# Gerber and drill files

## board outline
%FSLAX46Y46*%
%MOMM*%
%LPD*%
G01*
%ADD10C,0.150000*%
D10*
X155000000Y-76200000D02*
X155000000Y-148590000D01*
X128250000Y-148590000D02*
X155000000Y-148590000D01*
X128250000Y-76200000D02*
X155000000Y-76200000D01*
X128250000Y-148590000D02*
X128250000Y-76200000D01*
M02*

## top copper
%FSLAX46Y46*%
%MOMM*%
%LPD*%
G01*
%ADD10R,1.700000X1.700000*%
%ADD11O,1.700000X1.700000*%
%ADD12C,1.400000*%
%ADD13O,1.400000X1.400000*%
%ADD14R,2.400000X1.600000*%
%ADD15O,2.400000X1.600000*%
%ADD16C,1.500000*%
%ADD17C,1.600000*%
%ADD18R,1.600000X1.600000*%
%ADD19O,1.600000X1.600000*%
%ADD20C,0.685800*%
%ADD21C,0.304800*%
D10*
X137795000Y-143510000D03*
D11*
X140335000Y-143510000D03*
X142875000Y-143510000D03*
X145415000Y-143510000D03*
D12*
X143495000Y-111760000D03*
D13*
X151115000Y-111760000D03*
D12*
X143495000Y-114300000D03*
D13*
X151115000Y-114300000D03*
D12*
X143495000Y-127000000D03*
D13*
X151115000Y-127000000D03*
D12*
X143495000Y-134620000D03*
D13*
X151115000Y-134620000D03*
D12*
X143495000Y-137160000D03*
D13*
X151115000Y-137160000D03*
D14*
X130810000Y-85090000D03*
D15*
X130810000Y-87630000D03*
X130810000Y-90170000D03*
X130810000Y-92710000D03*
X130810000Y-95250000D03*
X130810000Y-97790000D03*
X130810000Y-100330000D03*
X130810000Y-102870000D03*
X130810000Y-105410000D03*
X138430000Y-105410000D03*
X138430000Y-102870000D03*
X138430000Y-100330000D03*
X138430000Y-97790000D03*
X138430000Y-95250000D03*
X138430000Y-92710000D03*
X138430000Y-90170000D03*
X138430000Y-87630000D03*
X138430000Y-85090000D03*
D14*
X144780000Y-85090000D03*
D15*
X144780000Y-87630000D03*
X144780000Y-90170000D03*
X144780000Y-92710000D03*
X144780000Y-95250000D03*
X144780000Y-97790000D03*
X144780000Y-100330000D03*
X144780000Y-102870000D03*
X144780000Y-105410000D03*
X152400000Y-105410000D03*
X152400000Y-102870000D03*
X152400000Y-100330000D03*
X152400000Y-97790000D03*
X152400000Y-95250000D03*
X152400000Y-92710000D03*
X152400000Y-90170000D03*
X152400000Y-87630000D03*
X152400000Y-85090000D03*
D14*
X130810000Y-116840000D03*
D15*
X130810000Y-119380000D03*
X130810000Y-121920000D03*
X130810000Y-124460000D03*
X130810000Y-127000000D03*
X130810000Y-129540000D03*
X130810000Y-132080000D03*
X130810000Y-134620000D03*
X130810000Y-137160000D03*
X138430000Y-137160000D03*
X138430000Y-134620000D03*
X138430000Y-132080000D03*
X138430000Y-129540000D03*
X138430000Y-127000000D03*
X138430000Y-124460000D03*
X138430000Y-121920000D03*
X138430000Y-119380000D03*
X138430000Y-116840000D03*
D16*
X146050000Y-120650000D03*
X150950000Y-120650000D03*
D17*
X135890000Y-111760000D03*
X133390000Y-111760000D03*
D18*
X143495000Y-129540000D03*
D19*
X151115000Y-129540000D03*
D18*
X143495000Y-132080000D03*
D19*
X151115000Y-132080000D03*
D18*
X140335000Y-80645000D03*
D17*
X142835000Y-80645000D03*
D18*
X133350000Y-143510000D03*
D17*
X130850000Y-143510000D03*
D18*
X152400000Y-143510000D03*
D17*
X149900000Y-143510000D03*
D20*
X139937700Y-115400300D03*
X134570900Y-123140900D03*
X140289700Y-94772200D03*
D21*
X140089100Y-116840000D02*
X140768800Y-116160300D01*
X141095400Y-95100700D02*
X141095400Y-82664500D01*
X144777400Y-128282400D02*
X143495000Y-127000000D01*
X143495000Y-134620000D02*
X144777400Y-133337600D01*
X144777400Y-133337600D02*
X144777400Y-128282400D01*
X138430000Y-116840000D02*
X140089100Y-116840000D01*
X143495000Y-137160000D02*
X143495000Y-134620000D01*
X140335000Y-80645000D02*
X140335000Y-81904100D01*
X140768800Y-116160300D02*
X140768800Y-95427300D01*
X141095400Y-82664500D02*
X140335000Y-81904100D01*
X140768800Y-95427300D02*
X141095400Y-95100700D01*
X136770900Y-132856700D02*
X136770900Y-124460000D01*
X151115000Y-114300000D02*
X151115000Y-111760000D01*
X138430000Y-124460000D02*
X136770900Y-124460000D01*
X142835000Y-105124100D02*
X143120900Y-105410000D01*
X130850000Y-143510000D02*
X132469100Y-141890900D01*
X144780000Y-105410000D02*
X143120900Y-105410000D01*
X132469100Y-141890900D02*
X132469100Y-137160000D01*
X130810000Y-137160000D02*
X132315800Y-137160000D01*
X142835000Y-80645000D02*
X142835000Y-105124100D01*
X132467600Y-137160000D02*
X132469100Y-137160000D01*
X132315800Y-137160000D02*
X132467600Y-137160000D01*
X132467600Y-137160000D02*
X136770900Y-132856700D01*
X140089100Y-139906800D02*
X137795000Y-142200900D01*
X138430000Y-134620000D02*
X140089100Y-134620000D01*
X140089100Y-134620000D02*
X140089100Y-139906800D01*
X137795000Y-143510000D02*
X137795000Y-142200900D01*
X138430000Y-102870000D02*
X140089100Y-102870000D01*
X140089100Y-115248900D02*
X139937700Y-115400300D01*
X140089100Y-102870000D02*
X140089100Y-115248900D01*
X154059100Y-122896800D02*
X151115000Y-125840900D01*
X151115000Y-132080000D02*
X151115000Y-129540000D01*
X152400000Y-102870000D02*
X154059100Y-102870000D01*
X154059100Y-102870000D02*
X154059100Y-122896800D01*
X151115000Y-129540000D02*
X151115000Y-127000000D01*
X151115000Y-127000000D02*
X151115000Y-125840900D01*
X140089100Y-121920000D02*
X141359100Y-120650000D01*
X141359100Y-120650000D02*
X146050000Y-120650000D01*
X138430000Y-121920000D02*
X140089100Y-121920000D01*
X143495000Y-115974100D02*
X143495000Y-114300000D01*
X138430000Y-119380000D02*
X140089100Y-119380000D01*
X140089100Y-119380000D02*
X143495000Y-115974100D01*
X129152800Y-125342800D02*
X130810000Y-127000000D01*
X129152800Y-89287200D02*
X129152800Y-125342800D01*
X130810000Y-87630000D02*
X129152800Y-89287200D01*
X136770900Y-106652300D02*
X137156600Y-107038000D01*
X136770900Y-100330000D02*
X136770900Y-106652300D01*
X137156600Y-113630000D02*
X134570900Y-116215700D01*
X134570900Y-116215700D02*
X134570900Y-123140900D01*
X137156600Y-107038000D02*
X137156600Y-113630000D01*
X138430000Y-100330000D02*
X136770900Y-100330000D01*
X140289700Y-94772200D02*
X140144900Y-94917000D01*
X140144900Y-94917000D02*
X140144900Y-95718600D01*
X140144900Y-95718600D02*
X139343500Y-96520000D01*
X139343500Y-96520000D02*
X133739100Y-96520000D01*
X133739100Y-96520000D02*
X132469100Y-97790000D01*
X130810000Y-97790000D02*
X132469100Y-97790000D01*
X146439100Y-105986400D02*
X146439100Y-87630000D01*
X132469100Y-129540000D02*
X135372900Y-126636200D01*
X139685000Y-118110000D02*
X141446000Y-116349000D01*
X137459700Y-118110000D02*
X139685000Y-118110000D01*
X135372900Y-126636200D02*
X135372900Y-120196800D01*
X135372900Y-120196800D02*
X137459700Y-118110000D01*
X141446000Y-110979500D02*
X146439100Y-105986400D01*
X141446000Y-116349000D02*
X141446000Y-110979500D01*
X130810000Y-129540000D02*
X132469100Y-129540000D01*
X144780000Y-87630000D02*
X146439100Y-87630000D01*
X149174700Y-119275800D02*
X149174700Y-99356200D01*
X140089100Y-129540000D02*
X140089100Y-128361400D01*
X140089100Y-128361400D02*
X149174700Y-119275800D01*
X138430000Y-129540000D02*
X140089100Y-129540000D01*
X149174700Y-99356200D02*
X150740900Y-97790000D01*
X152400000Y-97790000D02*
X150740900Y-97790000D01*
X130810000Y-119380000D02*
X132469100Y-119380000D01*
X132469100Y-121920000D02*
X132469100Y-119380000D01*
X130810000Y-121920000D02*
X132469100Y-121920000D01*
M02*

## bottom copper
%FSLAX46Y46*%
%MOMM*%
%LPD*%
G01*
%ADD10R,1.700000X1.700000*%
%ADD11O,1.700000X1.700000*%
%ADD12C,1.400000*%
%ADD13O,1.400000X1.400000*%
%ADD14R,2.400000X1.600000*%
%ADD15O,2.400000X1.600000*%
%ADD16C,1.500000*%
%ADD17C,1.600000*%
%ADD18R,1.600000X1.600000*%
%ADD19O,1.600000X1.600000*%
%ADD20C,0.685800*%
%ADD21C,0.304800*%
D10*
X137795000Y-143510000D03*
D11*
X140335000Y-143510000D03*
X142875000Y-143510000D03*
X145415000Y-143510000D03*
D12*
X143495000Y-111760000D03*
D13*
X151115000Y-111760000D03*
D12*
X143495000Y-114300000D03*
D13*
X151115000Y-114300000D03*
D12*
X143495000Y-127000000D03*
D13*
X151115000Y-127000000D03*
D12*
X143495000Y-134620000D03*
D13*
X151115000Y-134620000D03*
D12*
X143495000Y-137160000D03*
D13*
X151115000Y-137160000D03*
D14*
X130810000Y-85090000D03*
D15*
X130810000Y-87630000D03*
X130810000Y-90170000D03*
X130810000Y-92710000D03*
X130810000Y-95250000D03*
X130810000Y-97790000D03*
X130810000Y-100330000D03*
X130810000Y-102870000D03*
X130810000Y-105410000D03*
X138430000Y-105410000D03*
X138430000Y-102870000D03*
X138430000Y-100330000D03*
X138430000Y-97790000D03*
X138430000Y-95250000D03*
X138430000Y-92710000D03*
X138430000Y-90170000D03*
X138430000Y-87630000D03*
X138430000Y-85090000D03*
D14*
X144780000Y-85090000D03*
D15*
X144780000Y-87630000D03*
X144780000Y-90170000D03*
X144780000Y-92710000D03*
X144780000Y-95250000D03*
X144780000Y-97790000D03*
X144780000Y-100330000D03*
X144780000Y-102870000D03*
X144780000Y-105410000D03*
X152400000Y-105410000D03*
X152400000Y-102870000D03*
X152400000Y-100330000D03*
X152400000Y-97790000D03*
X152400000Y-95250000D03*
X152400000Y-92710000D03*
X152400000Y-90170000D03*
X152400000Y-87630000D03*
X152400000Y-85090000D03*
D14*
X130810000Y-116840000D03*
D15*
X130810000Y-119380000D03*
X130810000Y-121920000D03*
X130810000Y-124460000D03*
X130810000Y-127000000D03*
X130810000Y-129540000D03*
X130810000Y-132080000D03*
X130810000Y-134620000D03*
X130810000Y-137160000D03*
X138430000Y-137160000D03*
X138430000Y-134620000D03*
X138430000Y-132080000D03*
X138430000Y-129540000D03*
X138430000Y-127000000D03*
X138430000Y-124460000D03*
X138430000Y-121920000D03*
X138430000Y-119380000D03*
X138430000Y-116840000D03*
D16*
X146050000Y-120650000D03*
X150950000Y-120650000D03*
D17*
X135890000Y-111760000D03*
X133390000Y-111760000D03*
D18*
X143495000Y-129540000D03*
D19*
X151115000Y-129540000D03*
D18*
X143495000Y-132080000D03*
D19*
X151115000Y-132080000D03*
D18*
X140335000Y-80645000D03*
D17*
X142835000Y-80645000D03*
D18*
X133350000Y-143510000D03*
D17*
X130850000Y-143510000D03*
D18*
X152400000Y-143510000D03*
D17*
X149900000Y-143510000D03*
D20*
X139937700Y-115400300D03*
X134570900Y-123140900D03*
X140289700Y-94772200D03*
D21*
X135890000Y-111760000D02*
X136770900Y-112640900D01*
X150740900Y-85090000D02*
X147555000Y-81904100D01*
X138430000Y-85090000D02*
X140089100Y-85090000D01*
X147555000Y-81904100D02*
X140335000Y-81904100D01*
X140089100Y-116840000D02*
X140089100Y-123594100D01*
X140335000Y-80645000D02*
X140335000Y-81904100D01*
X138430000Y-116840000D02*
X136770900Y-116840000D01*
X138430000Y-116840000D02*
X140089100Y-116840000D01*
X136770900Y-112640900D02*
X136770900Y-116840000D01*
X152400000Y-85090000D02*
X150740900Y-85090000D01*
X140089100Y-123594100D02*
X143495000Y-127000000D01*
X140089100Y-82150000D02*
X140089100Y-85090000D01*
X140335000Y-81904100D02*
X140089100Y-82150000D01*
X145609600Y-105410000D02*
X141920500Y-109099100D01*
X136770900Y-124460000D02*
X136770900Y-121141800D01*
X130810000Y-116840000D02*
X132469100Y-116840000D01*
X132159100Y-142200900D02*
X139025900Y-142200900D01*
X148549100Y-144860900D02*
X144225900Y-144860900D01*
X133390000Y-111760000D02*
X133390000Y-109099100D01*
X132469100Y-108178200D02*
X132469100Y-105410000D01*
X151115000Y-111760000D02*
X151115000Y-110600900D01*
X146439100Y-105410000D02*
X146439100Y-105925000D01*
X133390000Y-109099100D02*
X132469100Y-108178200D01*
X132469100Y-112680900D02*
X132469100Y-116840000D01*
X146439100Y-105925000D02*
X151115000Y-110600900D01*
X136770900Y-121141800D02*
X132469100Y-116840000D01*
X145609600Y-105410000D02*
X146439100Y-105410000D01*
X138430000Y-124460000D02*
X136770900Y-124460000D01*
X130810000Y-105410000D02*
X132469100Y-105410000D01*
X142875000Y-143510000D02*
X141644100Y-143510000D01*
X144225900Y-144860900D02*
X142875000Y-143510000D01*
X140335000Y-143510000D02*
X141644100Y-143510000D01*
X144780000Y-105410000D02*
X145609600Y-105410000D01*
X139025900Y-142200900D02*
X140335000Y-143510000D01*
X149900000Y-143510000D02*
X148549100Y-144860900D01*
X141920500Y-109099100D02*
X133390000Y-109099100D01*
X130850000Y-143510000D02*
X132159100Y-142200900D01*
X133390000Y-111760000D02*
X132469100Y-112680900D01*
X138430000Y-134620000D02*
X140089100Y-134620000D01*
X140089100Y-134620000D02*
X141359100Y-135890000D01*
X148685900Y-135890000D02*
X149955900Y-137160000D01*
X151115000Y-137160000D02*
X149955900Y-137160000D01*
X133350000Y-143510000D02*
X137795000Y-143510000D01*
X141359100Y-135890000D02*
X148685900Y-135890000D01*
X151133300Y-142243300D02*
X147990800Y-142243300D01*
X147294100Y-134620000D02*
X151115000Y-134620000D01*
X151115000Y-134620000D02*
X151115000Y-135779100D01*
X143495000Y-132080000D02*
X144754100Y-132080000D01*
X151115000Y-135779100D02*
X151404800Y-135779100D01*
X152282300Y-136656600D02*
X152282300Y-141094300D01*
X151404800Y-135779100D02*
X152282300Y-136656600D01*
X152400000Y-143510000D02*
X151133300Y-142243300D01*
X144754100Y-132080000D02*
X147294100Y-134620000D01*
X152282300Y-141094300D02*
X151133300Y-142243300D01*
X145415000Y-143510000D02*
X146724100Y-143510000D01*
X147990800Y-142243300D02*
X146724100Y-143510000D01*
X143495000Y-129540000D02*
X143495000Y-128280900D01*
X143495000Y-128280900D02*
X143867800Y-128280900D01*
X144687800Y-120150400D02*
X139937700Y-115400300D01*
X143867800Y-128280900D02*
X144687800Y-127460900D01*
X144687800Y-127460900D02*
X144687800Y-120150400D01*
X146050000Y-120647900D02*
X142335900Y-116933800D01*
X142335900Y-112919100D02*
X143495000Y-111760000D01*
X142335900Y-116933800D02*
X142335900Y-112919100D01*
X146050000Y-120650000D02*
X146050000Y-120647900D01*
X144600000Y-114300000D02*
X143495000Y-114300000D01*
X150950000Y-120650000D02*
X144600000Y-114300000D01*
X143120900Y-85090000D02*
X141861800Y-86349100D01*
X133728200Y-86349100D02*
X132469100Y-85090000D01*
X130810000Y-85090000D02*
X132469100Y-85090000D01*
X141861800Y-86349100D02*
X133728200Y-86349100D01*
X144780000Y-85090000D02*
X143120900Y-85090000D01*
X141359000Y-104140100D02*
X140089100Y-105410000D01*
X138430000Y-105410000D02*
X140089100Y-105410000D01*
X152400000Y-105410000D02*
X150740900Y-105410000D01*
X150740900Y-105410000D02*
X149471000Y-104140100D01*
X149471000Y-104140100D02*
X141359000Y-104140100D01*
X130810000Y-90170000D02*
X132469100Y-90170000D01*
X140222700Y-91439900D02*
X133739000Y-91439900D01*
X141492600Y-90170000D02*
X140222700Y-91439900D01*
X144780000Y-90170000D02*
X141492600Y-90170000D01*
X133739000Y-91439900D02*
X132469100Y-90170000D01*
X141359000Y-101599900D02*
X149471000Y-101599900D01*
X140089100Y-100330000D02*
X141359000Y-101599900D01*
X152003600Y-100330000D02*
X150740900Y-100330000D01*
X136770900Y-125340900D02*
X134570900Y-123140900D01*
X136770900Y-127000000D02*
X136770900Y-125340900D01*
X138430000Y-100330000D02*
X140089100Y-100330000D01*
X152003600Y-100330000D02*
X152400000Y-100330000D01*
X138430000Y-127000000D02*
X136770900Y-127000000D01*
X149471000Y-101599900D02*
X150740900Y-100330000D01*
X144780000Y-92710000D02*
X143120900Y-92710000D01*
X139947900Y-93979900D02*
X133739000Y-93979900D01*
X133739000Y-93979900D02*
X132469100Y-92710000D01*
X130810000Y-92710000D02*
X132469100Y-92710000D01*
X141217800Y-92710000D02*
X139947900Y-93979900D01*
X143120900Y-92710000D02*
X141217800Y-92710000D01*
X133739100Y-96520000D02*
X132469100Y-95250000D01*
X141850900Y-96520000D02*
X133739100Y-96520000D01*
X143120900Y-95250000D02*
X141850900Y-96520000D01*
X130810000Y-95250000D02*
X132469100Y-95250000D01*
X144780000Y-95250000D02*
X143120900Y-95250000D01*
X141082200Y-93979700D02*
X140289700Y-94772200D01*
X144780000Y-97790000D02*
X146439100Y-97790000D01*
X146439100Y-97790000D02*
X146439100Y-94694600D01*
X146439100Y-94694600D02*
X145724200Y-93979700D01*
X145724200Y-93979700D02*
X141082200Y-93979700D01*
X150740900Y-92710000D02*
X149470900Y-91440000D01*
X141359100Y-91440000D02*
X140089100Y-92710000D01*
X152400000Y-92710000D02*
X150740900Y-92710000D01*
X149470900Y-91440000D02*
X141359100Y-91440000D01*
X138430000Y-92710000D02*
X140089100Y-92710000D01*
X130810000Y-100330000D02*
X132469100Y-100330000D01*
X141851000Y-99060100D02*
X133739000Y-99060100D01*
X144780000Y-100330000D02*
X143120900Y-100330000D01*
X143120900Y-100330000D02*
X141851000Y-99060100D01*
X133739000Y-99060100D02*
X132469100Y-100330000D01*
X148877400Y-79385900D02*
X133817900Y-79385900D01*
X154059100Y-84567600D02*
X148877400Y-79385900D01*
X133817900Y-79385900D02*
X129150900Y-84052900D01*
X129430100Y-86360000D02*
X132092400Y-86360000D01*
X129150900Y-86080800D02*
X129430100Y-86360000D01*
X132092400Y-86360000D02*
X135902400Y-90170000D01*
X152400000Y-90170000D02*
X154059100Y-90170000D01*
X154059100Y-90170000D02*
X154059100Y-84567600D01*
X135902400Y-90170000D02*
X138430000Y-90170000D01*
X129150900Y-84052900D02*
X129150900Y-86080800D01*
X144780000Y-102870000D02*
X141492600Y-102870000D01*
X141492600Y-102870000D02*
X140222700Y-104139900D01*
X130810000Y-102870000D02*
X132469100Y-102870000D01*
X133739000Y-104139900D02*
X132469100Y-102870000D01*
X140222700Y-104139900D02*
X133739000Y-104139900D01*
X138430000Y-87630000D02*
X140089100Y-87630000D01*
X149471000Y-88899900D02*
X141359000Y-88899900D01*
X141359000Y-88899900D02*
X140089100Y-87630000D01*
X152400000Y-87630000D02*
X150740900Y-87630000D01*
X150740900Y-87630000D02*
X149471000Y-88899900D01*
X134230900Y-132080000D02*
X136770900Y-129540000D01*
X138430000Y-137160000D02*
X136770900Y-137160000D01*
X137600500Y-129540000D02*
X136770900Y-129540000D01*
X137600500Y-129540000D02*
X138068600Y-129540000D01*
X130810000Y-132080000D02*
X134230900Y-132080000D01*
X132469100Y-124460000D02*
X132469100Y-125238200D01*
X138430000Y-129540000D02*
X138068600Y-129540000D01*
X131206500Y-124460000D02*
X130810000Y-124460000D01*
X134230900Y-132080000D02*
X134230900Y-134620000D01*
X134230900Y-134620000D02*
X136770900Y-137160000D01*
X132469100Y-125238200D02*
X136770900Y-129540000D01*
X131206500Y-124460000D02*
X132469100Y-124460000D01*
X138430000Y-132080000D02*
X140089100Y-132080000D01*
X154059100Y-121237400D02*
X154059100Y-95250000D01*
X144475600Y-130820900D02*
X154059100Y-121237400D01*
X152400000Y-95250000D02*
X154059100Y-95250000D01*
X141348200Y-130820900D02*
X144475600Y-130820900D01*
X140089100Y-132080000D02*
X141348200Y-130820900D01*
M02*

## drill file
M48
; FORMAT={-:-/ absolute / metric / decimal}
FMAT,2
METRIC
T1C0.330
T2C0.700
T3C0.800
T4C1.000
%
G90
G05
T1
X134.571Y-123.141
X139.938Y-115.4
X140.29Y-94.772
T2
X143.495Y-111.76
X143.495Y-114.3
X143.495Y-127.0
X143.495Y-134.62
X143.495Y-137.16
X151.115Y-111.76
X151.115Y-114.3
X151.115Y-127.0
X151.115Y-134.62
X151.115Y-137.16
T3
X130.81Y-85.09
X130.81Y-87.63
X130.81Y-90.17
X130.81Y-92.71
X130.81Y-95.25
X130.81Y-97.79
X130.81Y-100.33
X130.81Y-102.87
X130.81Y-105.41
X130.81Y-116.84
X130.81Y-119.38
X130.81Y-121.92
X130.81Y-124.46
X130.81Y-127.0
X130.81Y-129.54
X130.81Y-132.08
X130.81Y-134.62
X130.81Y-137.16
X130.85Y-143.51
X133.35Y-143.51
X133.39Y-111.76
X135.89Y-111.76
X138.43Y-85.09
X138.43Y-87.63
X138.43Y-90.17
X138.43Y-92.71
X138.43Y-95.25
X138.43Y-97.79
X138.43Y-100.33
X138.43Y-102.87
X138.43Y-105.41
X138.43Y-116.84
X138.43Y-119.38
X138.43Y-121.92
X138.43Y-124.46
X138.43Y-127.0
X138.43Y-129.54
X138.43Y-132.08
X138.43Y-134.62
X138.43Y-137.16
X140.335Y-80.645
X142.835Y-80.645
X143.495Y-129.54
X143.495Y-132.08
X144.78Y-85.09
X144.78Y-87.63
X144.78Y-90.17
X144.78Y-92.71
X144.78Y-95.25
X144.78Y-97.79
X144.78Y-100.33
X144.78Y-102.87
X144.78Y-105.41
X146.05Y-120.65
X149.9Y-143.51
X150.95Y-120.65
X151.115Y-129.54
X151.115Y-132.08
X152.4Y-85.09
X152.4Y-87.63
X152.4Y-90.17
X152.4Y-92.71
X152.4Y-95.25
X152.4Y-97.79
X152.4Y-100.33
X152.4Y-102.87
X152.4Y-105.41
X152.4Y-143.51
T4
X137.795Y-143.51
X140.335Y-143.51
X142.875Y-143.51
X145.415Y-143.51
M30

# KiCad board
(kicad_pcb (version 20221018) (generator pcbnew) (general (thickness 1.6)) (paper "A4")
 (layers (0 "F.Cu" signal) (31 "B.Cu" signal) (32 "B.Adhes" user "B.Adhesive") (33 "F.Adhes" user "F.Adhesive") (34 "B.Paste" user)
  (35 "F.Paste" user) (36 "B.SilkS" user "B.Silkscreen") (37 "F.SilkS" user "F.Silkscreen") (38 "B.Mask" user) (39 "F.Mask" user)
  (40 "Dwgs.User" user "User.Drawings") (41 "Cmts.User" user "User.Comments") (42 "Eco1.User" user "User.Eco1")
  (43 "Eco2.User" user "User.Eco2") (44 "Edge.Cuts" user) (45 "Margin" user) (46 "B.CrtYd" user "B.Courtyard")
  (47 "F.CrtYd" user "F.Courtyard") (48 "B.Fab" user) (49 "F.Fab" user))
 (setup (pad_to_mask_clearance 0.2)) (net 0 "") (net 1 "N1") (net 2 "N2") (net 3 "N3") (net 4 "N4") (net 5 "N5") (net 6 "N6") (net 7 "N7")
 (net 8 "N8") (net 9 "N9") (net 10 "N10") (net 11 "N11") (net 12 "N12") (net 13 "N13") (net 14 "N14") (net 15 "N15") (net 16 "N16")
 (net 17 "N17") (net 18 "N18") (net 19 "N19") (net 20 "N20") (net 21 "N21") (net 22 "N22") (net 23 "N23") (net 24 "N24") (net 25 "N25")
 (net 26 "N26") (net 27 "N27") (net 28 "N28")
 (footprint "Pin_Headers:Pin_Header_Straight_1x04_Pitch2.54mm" (layer "F.Cu") (at 137.795 143.51 90)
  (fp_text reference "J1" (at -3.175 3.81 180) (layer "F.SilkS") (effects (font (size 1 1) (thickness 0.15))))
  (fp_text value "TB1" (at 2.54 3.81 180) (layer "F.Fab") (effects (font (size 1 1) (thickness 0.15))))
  (pad "1" thru_hole rect (at 0 0 90) (size 1.7 1.7) (drill 1) (layers "*.Cu" "*.Mask") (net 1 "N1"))
  (pad "2" thru_hole oval (at 0 2.54 90) (size 1.7 1.7) (drill 1) (layers "*.Cu" "*.Mask") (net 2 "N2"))
  (pad "3" thru_hole oval (at 0 5.08 90) (size 1.7 1.7) (drill 1) (layers "*.Cu" "*.Mask") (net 2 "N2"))
  (pad "4" thru_hole oval (at 0 7.62 90) (size 1.7 1.7) (drill 1) (layers "*.Cu" "*.Mask") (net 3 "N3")))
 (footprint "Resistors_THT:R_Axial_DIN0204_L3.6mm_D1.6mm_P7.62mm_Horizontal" (layer "F.Cu") (at 143.495 111.76)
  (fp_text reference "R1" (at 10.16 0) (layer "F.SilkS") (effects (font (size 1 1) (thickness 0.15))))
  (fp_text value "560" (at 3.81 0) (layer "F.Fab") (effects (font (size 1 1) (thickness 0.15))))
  (pad "1" thru_hole circle (at 0 0) (size 1.4 1.4) (drill 0.7) (layers "*.Cu" "*.Mask") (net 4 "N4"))
  (pad "2" thru_hole oval (at 7.62 0) (size 1.4 1.4) (drill 0.7) (layers "*.Cu" "*.Mask") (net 2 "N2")))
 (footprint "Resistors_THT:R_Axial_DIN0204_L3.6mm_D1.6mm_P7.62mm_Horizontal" (layer "F.Cu") (at 143.495 114.3)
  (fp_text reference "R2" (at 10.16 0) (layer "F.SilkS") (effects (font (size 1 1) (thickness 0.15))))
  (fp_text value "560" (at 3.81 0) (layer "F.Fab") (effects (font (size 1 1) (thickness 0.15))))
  (pad "1" thru_hole circle (at 0 0) (size 1.4 1.4) (drill 0.7) (layers "*.Cu" "*.Mask") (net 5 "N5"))
  (pad "2" thru_hole oval (at 7.62 0) (size 1.4 1.4) (drill 0.7) (layers "*.Cu" "*.Mask") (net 2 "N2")))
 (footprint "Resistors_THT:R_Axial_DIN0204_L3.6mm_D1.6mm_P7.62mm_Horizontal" (layer "F.Cu") (at 143.495 127)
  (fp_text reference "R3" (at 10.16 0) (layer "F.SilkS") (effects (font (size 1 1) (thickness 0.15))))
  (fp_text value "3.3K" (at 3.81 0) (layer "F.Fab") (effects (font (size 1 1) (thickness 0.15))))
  (pad "1" thru_hole circle (at 0 0) (size 1.4 1.4) (drill 0.7) (layers "*.Cu" "*.Mask") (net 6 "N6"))
  (pad "2" thru_hole oval (at 7.62 0) (size 1.4 1.4) (drill 0.7) (layers "*.Cu" "*.Mask") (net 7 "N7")))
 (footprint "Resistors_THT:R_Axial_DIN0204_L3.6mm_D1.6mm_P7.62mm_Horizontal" (layer "F.Cu") (at 143.495 134.62)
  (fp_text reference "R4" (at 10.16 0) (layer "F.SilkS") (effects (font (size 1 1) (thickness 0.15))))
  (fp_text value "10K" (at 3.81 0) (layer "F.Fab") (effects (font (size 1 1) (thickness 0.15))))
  (pad "1" thru_hole circle (at 0 0) (size 1.4 1.4) (drill 0.7) (layers "*.Cu" "*.Mask") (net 6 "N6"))
  (pad "2" thru_hole oval (at 7.62 0) (size 1.4 1.4) (drill 0.7) (layers "*.Cu" "*.Mask") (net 3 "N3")))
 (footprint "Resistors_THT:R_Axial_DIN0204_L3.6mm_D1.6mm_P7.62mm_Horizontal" (layer "F.Cu") (at 143.495 137.16)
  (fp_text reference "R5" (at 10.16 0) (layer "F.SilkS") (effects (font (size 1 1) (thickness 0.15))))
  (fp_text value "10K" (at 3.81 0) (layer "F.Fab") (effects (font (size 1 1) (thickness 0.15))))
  (pad "1" thru_hole circle (at 0 0) (size 1.4 1.4) (drill 0.7) (layers "*.Cu" "*.Mask") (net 6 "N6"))
  (pad "2" thru_hole oval (at 7.62 0) (size 1.4 1.4) (drill 0.7) (layers "*.Cu" "*.Mask") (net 1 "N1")))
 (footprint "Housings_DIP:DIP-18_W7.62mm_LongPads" (layer "F.Cu") (at 130.81 85.09)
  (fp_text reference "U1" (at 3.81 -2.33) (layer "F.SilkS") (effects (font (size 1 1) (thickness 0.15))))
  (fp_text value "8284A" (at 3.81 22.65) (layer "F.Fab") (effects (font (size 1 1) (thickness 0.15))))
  (pad "1" thru_hole rect (at 0 0) (size 2.4 1.6) (drill 0.8) (layers "*.Cu" "*.Mask") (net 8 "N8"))
  (pad "2" thru_hole oval (at 0 2.54) (size 2.4 1.6) (drill 0.8) (layers "*.Cu" "*.Mask") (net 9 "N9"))
  (pad "3" thru_hole oval (at 0 5.08) (size 2.4 1.6) (drill 0.8) (layers "*.Cu" "*.Mask") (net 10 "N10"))
  (pad "4" thru_hole oval (at 0 7.62) (size 2.4 1.6) (drill 0.8) (layers "*.Cu" "*.Mask") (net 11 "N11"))
  (pad "5" thru_hole oval (at 0 10.16) (size 2.4 1.6) (drill 0.8) (layers "*.Cu" "*.Mask") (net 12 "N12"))
  (pad "6" thru_hole oval (at 0 12.7) (size 2.4 1.6) (drill 0.8) (layers "*.Cu" "*.Mask") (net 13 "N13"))
  (pad "7" thru_hole oval (at 0 15.24) (size 2.4 1.6) (drill 0.8) (layers "*.Cu" "*.Mask") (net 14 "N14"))
  (pad "8" thru_hole oval (at 0 17.78) (size 2.4 1.6) (drill 0.8) (layers "*.Cu" "*.Mask") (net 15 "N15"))
  (pad "9" thru_hole oval (at 0 20.32) (size 2.4 1.6) (drill 0.8) (layers "*.Cu" "*.Mask") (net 2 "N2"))
  (pad "10" thru_hole oval (at 7.62 20.32) (size 2.4 1.6) (drill 0.8) (layers "*.Cu" "*.Mask") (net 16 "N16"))
  (pad "11" thru_hole oval (at 7.62 17.78) (size 2.4 1.6) (drill 0.8) (layers "*.Cu" "*.Mask") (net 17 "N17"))
  (pad "12" thru_hole oval (at 7.62 15.24) (size 2.4 1.6) (drill 0.8) (layers "*.Cu" "*.Mask") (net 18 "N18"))
  (pad "13" thru_hole oval (at 7.62 12.7) (size 2.4 1.6) (drill 0.8) (layers "*.Cu" "*.Mask") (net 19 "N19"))
  (pad "14" thru_hole oval (at 7.62 10.16) (size 2.4 1.6) (drill 0.8) (layers "*.Cu" "*.Mask") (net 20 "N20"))
  (pad "15" thru_hole oval (at 7.62 7.62) (size 2.4 1.6) (drill 0.8) (layers "*.Cu" "*.Mask") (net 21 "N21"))
  (pad "16" thru_hole oval (at 7.62 5.08) (size 2.4 1.6) (drill 0.8) (layers "*.Cu" "*.Mask") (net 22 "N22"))
  (pad "17" thru_hole oval (at 7.62 2.54) (size 2.4 1.6) (drill 0.8) (layers "*.Cu" "*.Mask") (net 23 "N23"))
  (pad "18" thru_hole oval (at 7.62 0) (size 2.4 1.6) (drill 0.8) (layers "*.Cu" "*.Mask") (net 6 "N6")))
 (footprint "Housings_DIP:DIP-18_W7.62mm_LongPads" (layer "F.Cu") (at 144.78 85.09)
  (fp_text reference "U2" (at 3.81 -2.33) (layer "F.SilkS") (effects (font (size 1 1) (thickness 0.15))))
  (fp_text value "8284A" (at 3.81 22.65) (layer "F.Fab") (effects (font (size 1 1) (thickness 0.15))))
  (pad "1" thru_hole rect (at 0 0) (size 2.4 1.6) (drill 0.8) (layers "*.Cu" "*.Mask") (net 8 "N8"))
  (pad "2" thru_hole oval (at 0 2.54) (size 2.4 1.6) (drill 0.8) (layers "*.Cu" "*.Mask") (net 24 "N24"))
  (pad "3" thru_hole oval (at 0 5.08) (size 2.4 1.6) (drill 0.8) (layers "*.Cu" "*.Mask") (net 10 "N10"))
  (pad "4" thru_hole oval (at 0 7.62) (size 2.4 1.6) (drill 0.8) (layers "*.Cu" "*.Mask") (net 11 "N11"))
  (pad "5" thru_hole oval (at 0 10.16) (size 2.4 1.6) (drill 0.8) (layers "*.Cu" "*.Mask") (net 12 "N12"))
  (pad "6" thru_hole oval (at 0 12.7) (size 2.4 1.6) (drill 0.8) (layers "*.Cu" "*.Mask") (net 13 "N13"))
  (pad "7" thru_hole oval (at 0 15.24) (size 2.4 1.6) (drill 0.8) (layers "*.Cu" "*.Mask") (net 14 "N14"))
  (pad "8" thru_hole oval (at 0 17.78) (size 2.4 1.6) (drill 0.8) (layers "*.Cu" "*.Mask") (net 15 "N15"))
  (pad "9" thru_hole oval (at 0 20.32) (size 2.4 1.6) (drill 0.8) (layers "*.Cu" "*.Mask") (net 2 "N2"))
  (pad "10" thru_hole oval (at 7.62 20.32) (size 2.4 1.6) (drill 0.8) (layers "*.Cu" "*.Mask") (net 16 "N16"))
  (pad "11" thru_hole oval (at 7.62 17.78) (size 2.4 1.6) (drill 0.8) (layers "*.Cu" "*.Mask") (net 7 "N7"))
  (pad "12" thru_hole oval (at 7.62 15.24) (size 2.4 1.6) (drill 0.8) (layers "*.Cu" "*.Mask") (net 18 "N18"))
  (pad "13" thru_hole oval (at 7.62 12.7) (size 2.4 1.6) (drill 0.8) (layers "*.Cu" "*.Mask") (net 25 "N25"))
  (pad "14" thru_hole oval (at 7.62 10.16) (size 2.4 1.6) (drill 0.8) (layers "*.Cu" "*.Mask") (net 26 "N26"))
  (pad "15" thru_hole oval (at 7.62 7.62) (size 2.4 1.6) (drill 0.8) (layers "*.Cu" "*.Mask") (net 21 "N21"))
  (pad "16" thru_hole oval (at 7.62 5.08) (size 2.4 1.6) (drill 0.8) (layers "*.Cu" "*.Mask") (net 22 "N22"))
  (pad "17" thru_hole oval (at 7.62 2.54) (size 2.4 1.6) (drill 0.8) (layers "*.Cu" "*.Mask") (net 23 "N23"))
  (pad "18" thru_hole oval (at 7.62 0) (size 2.4 1.6) (drill 0.8) (layers "*.Cu" "*.Mask") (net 6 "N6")))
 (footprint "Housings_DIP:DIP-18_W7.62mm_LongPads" (layer "F.Cu") (at 130.81 116.84)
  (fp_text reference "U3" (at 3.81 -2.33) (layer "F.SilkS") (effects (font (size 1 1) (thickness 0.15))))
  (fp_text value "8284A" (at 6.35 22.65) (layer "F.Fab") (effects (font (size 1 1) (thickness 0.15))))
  (pad "1" thru_hole rect (at 0 0) (size 2.4 1.6) (drill 0.8) (layers "*.Cu" "*.Mask") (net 2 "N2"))
  (pad "2" thru_hole oval (at 0 2.54) (size 2.4 1.6) (drill 0.8) (layers "*.Cu" "*.Mask") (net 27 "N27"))
  (pad "3" thru_hole oval (at 0 5.08) (size 2.4 1.6) (drill 0.8) (layers "*.Cu" "*.Mask") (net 27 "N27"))
  (pad "4" thru_hole oval (at 0 7.62) (size 2.4 1.6) (drill 0.8) (layers "*.Cu" "*.Mask") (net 25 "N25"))
  (pad "5" thru_hole oval (at 0 10.16) (size 2.4 1.6) (drill 0.8) (layers "*.Cu" "*.Mask") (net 9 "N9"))
  (pad "6" thru_hole oval (at 0 12.7) (size 2.4 1.6) (drill 0.8) (layers "*.Cu" "*.Mask") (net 24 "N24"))
  (pad "7" thru_hole oval (at 0 15.24) (size 2.4 1.6) (drill 0.8) (layers "*.Cu" "*.Mask") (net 25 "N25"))
  (pad "8" thru_hole oval (at 0 17.78) (size 2.4 1.6) (drill 0.8) (layers "*.Cu" "*.Mask") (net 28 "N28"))
  (pad "9" thru_hole oval (at 0 20.32) (size 2.4 1.6) (drill 0.8) (layers "*.Cu" "*.Mask") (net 2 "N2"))
  (pad "10" thru_hole oval (at 7.62 20.32) (size 2.4 1.6) (drill 0.8) (layers "*.Cu" "*.Mask") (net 25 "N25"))
  (pad "11" thru_hole oval (at 7.62 17.78) (size 2.4 1.6) (drill 0.8) (layers "*.Cu" "*.Mask") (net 1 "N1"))
  (pad "12" thru_hole oval (at 7.62 15.24) (size 2.4 1.6) (drill 0.8) (layers "*.Cu" "*.Mask") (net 26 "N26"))
  (pad "13" thru_hole oval (at 7.62 12.7) (size 2.4 1.6) (drill 0.8) (layers "*.Cu" "*.Mask") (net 25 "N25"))
  (pad "14" thru_hole oval (at 7.62 10.16) (size 2.4 1.6) (drill 0.8) (layers "*.Cu" "*.Mask") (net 18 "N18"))
  (pad "15" thru_hole oval (at 7.62 7.62) (size 2.4 1.6) (drill 0.8) (layers "*.Cu" "*.Mask") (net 2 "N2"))
  (pad "16" thru_hole oval (at 7.62 5.08) (size 2.4 1.6) (drill 0.8) (layers "*.Cu" "*.Mask") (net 4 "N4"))
  (pad "17" thru_hole oval (at 7.62 2.54) (size 2.4 1.6) (drill 0.8) (layers "*.Cu" "*.Mask") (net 5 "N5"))
  (pad "18" thru_hole oval (at 7.62 0) (size 2.4 1.6) (drill 0.8) (layers "*.Cu" "*.Mask") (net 6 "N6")))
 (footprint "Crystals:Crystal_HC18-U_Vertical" (layer "F.Cu") (at 146.05 120.65)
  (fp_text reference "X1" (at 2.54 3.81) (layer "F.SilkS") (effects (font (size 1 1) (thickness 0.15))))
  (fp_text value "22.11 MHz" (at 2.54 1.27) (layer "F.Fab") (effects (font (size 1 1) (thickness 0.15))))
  (pad "1" thru_hole circle (at 0 0) (size 1.5 1.5) (drill 0.8) (layers "*.Cu" "*.Mask") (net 4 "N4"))
  (pad "2" thru_hole circle (at 4.9 0) (size 1.5 1.5) (drill 0.8) (layers "*.Cu" "*.Mask") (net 5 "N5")))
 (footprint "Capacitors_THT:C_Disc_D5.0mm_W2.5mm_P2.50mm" (layer "F.Cu") (at 135.89 111.76 180)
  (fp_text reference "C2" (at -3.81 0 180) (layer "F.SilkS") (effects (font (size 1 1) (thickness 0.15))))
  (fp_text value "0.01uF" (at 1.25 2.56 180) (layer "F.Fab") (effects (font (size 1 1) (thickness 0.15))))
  (pad "1" thru_hole circle (at 0 0 180) (size 1.6 1.6) (drill 0.8) (layers "*.Cu" "*.Mask") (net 6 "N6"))
  (pad "2" thru_hole circle (at 2.5 0 180) (size 1.6 1.6) (drill 0.8) (layers "*.Cu" "*.Mask") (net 2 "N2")))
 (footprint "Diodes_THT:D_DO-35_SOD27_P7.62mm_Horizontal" (layer "F.Cu") (at 143.495 129.54)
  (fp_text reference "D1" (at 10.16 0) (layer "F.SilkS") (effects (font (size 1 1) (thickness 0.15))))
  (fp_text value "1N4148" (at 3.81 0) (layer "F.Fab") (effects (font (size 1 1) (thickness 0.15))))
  (pad "1" thru_hole rect (at 0 0) (size 1.6 1.6) (drill 0.8) (layers "*.Cu" "*.Mask") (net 17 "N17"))
  (pad "2" thru_hole oval (at 7.62 0) (size 1.6 1.6) (drill 0.8) (layers "*.Cu" "*.Mask") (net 7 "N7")))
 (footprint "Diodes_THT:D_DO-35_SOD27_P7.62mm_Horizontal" (layer "F.Cu") (at 143.495 132.08)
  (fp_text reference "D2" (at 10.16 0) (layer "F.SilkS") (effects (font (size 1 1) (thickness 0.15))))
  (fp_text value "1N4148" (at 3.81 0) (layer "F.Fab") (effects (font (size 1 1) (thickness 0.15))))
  (pad "1" thru_hole rect (at 0 0) (size 1.6 1.6) (drill 0.8) (layers "*.Cu" "*.Mask") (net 3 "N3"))
  (pad "2" thru_hole oval (at 7.62 0) (size 1.6 1.6) (drill 0.8) (layers "*.Cu" "*.Mask") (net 7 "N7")))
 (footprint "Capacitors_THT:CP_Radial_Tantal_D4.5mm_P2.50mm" (layer "F.Cu") (at 140.335 80.645)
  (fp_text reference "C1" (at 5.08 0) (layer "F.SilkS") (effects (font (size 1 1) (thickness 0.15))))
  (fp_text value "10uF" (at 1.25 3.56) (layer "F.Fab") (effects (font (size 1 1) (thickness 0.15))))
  (pad "1" thru_hole rect (at 0 0) (size 1.6 1.6) (drill 0.8) (layers "*.Cu" "*.Mask") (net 6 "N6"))
  (pad "2" thru_hole circle (at 2.5 0) (size 1.6 1.6) (drill 0.8) (layers "*.Cu" "*.Mask") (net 2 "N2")))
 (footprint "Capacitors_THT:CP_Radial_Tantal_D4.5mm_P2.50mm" (layer "F.Cu") (at 133.35 143.51 180)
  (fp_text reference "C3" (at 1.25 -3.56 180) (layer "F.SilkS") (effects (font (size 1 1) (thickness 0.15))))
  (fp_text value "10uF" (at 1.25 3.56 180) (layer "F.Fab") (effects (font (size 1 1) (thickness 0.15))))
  (pad "1" thru_hole rect (at 0 0 180) (size 1.6 1.6) (drill 0.8) (layers "*.Cu" "*.Mask") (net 1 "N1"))
  (pad "2" thru_hole circle (at 2.5 0 180) (size 1.6 1.6) (drill 0.8) (layers "*.Cu" "*.Mask") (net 2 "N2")))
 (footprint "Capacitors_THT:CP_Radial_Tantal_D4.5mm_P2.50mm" (layer "F.Cu") (at 152.4 143.51 180)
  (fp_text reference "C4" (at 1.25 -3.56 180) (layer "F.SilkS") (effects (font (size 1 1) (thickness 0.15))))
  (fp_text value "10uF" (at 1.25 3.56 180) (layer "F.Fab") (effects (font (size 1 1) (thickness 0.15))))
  (pad "1" thru_hole rect (at 0 0 180) (size 1.6 1.6) (drill 0.8) (layers "*.Cu" "*.Mask") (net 3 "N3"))
  (pad "2" thru_hole circle (at 2.5 0 180) (size 1.6 1.6) (drill 0.8) (layers "*.Cu" "*.Mask") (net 2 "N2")))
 (gr_line (start 155 76.2) (end 155 148.59) (stroke (width 0.15) (type solid)) (layer "Edge.Cuts"))
 (gr_line (start 128.25 148.59) (end 155 148.59) (stroke (width 0.15) (type default)) (layer "Edge.Cuts"))
 (gr_line (start 128.25 76.2) (end 155 76.2) (stroke (width 0.15) (type default)) (layer "Edge.Cuts"))
 (gr_line (start 128.25 148.59) (end 128.25 76.2) (stroke (width 0.15) (type solid)) (layer "Edge.Cuts"))
 (segment (start 140.0891 116.84) (end 140.7688 116.1603) (width 0.3048) (layer "F.Cu") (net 6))
 (segment (start 141.0954 95.1007) (end 141.0954 82.6645) (width 0.3048) (layer "F.Cu") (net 6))
 (segment (start 144.7774 128.2824) (end 143.495 127) (width 0.3048) (layer "F.Cu") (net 6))
 (segment (start 143.495 134.62) (end 144.7774 133.3376) (width 0.3048) (layer "F.Cu") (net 6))
 (segment (start 144.7774 133.3376) (end 144.7774 128.2824) (width 0.3048) (layer "F.Cu") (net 6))
 (segment (start 138.43 116.84) (end 140.0891 116.84) (width 0.3048) (layer "F.Cu") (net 6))
 (segment (start 143.495 137.16) (end 143.495 134.62) (width 0.3048) (layer "F.Cu") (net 6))
 (segment (start 140.335 80.645) (end 140.335 81.9041) (width 0.3048) (layer "F.Cu") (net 6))
 (segment (start 140.7688 116.1603) (end 140.7688 95.4273) (width 0.3048) (layer "F.Cu") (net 6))
 (segment (start 141.0954 82.6645) (end 140.335 81.9041) (width 0.3048) (layer "F.Cu") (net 6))
 (segment (start 140.7688 95.4273) (end 141.0954 95.1007) (width 0.3048) (layer "F.Cu") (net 6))
 (segment (start 135.89 111.76) (end 136.7709 112.6409) (width 0.3048) (layer "B.Cu") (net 6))
 (segment (start 150.7409 85.09) (end 147.555 81.9041) (width 0.3048) (layer "B.Cu") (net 6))
 (segment (start 138.43 85.09) (end 140.0891 85.09) (width 0.3048) (layer "B.Cu") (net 6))
 (segment (start 147.555 81.9041) (end 140.335 81.9041) (width 0.3048) (layer "B.Cu") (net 6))
 (segment (start 140.0891 116.84) (end 140.0891 123.5941) (width 0.3048) (layer "B.Cu") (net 6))
 (segment (start 140.335 80.645) (end 140.335 81.9041) (width 0.3048) (layer "B.Cu") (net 6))
 (segment (start 138.43 116.84) (end 136.7709 116.84) (width 0.3048) (layer "B.Cu") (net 6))
 (segment (start 138.43 116.84) (end 140.0891 116.84) (width 0.3048) (layer "B.Cu") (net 6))
 (segment (start 136.7709 112.6409) (end 136.7709 116.84) (width 0.3048) (layer "B.Cu") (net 6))
 (segment (start 152.4 85.09) (end 150.7409 85.09) (width 0.3048) (layer "B.Cu") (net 6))
 (segment (start 140.0891 123.5941) (end 143.495 127) (width 0.3048) (layer "B.Cu") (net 6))
 (segment (start 140.0891 82.15) (end 140.0891 85.09) (width 0.3048) (layer "B.Cu") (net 6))
 (segment (start 140.335 81.9041) (end 140.0891 82.15) (width 0.3048) (layer "B.Cu") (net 6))
 (segment (start 136.7709 132.8567) (end 136.7709 124.46) (width 0.3048) (layer "F.Cu") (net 2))
 (segment (start 151.115 114.3) (end 151.115 111.76) (width 0.3048) (layer "F.Cu") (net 2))
 (segment (start 138.43 124.46) (end 136.7709 124.46) (width 0.3048) (layer "F.Cu") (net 2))
 (segment (start 142.835 105.1241) (end 143.1209 105.41) (width 0.3048) (layer "F.Cu") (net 2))
 (segment (start 130.85 143.51) (end 132.4691 141.8909) (width 0.3048) (layer "F.Cu") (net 2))
 (segment (start 144.78 105.41) (end 143.1209 105.41) (width 0.3048) (layer "F.Cu") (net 2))
 (segment (start 132.4691 141.8909) (end 132.4691 137.16) (width 0.3048) (layer "F.Cu") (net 2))
 (segment (start 130.81 137.16) (end 132.3158 137.16) (width 0.3048) (layer "F.Cu") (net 2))
 (segment (start 142.835 80.645) (end 142.835 105.1241) (width 0.3048) (layer "F.Cu") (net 2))
 (segment (start 132.4676 137.16) (end 132.4691 137.16) (width 0.3048) (layer "F.Cu") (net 2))
 (segment (start 132.3158 137.16) (end 132.4676 137.16) (width 0.3048) (layer "F.Cu") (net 2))
 (segment (start 132.4676 137.16) (end 136.7709 132.8567) (width 0.3048) (layer "F.Cu") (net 2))
 (segment (start 145.6096 105.41) (end 141.9205 109.0991) (width 0.3048) (layer "B.Cu") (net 2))
 (segment (start 136.7709 124.46) (end 136.7709 121.1418) (width 0.3048) (layer "B.Cu") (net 2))
 (segment (start 130.81 116.84) (end 132.4691 116.84) (width 0.3048) (layer "B.Cu") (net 2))
 (segment (start 132.1591 142.2009) (end 139.0259 142.2009) (width 0.3048) (layer "B.Cu") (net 2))
 (segment (start 148.5491 144.8609) (end 144.2259 144.8609) (width 0.3048) (layer "B.Cu") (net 2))
 (segment (start 133.39 111.76) (end 133.39 109.0991) (width 0.3048) (layer "B.Cu") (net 2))
 (segment (start 132.4691 108.1782) (end 132.4691 105.41) (width 0.3048) (layer "B.Cu") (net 2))
 (segment (start 151.115 111.76) (end 151.115 110.6009) (width 0.3048) (layer "B.Cu") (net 2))
 (segment (start 146.4391 105.41) (end 146.4391 105.925) (width 0.3048) (layer "B.Cu") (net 2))
 (segment (start 133.39 109.0991) (end 132.4691 108.1782) (width 0.3048) (layer "B.Cu") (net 2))
 (segment (start 132.4691 112.6809) (end 132.4691 116.84) (width 0.3048) (layer "B.Cu") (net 2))
 (segment (start 146.4391 105.925) (end 151.115 110.6009) (width 0.3048) (layer "B.Cu") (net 2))
 (segment (start 136.7709 121.1418) (end 132.4691 116.84) (width 0.3048) (layer "B.Cu") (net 2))
 (segment (start 145.6096 105.41) (end 146.4391 105.41) (width 0.3048) (layer "B.Cu") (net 2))
 (segment (start 138.43 124.46) (end 136.7709 124.46) (width 0.3048) (layer "B.Cu") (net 2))
 (segment (start 130.81 105.41) (end 132.4691 105.41) (width 0.3048) (layer "B.Cu") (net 2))
 (segment (start 142.875 143.51) (end 141.6441 143.51) (width 0.3048) (layer "B.Cu") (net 2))
 (segment (start 144.2259 144.8609) (end 142.875 143.51) (width 0.3048) (layer "B.Cu") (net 2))
 (segment (start 140.335 143.51) (end 141.6441 143.51) (width 0.3048) (layer "B.Cu") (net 2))
 (segment (start 144.78 105.41) (end 145.6096 105.41) (width 0.3048) (layer "B.Cu") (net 2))
 (segment (start 139.0259 142.2009) (end 140.335 143.51) (width 0.3048) (layer "B.Cu") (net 2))
 (segment (start 149.9 143.51) (end 148.5491 144.8609) (width 0.3048) (layer "B.Cu") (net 2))
 (segment (start 141.9205 109.0991) (end 133.39 109.0991) (width 0.3048) (layer "B.Cu") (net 2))
 (segment (start 130.85 143.51) (end 132.1591 142.2009) (width 0.3048) (layer "B.Cu") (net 2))
 (segment (start 133.39 111.76) (end 132.4691 112.6809) (width 0.3048) (layer "B.Cu") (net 2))
 (segment (start 140.0891 139.9068) (end 137.795 142.2009) (width 0.3048) (layer "F.Cu") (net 1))
 (segment (start 138.43 134.62) (end 140.0891 134.62) (width 0.3048) (layer "F.Cu") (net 1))
 (segment (start 140.0891 134.62) (end 140.0891 139.9068) (width 0.3048) (layer "F.Cu") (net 1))
 (segment (start 137.795 143.51) (end 137.795 142.2009) (width 0.3048) (layer "F.Cu") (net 1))
 (segment (start 138.43 134.62) (end 140.0891 134.62) (width 0.3048) (layer "B.Cu") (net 1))
 (segment (start 140.0891 134.62) (end 141.3591 135.89) (width 0.3048) (layer "B.Cu") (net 1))
 (segment (start 148.6859 135.89) (end 149.9559 137.16) (width 0.3048) (layer "B.Cu") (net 1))
 (segment (start 151.115 137.16) (end 149.9559 137.16) (width 0.3048) (layer "B.Cu") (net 1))
 (segment (start 133.35 143.51) (end 137.795 143.51) (width 0.3048) (layer "B.Cu") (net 1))
 (segment (start 141.3591 135.89) (end 148.6859 135.89) (width 0.3048) (layer "B.Cu") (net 1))
 (segment (start 151.1333 142.2433) (end 147.9908 142.2433) (width 0.3048) (layer "B.Cu") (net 3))
 (segment (start 147.2941 134.62) (end 151.115 134.62) (width 0.3048) (layer "B.Cu") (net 3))
 (segment (start 151.115 134.62) (end 151.115 135.7791) (width 0.3048) (layer "B.Cu") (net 3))
 (segment (start 143.495 132.08) (end 144.7541 132.08) (width 0.3048) (layer "B.Cu") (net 3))
 (segment (start 151.115 135.7791) (end 151.4048 135.7791) (width 0.3048) (layer "B.Cu") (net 3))
 (segment (start 152.2823 136.6566) (end 152.2823 141.0943) (width 0.3048) (layer "B.Cu") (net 3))
 (segment (start 151.4048 135.7791) (end 152.2823 136.6566) (width 0.3048) (layer "B.Cu") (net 3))
 (segment (start 152.4 143.51) (end 151.1333 142.2433) (width 0.3048) (layer "B.Cu") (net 3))
 (segment (start 144.7541 132.08) (end 147.2941 134.62) (width 0.3048) (layer "B.Cu") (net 3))
 (segment (start 152.2823 141.0943) (end 151.1333 142.2433) (width 0.3048) (layer "B.Cu") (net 3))
 (segment (start 145.415 143.51) (end 146.7241 143.51) (width 0.3048) (layer "B.Cu") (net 3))
 (segment (start 147.9908 142.2433) (end 146.7241 143.51) (width 0.3048) (layer "B.Cu") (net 3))
 (segment (start 138.43 102.87) (end 140.0891 102.87) (width 0.3048) (layer "F.Cu") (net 17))
 (segment (start 140.0891 115.2489) (end 139.9377 115.4003) (width 0.3048) (layer "F.Cu") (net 17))
 (segment (start 140.0891 102.87) (end 140.0891 115.2489) (width 0.3048) (layer "F.Cu") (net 17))
 (via (at 139.9377 115.4003) (size 0.6858) (drill 0.3302) (layers "F.Cu" "B.Cu") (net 17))
 (segment (start 143.495 129.54) (end 143.495 128.2809) (width 0.3048) (layer "B.Cu") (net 17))
 (segment (start 143.495 128.2809) (end 143.8678 128.2809) (width 0.3048) (layer "B.Cu") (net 17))
 (segment (start 144.6878 120.1504) (end 139.9377 115.4003) (width 0.3048) (layer "B.Cu") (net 17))
 (segment (start 143.8678 128.2809) (end 144.6878 127.4609) (width 0.3048) (layer "B.Cu") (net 17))
 (segment (start 144.6878 127.4609) (end 144.6878 120.1504) (width 0.3048) (layer "B.Cu") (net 17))
 (segment (start 154.0591 122.8968) (end 151.115 125.8409) (width 0.3048) (layer "F.Cu") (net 7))
 (segment (start 151.115 132.08) (end 151.115 129.54) (width 0.3048) (layer "F.Cu") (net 7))
 (segment (start 152.4 102.87) (end 154.0591 102.87) (width 0.3048) (layer "F.Cu") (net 7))
 (segment (start 154.0591 102.87) (end 154.0591 122.8968) (width 0.3048) (layer "F.Cu") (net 7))
 (segment (start 151.115 129.54) (end 151.115 127) (width 0.3048) (layer "F.Cu") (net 7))
 (segment (start 151.115 127) (end 151.115 125.8409) (width 0.3048) (layer "F.Cu") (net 7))
 (segment (start 140.0891 121.92) (end 141.3591 120.65) (width 0.3048) (layer "F.Cu") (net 4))
 (segment (start 141.3591 120.65) (end 146.05 120.65) (width 0.3048) (layer "F.Cu") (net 4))
 (segment (start 138.43 121.92) (end 140.0891 121.92) (width 0.3048) (layer "F.Cu") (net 4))
 (segment (start 146.05 120.6479) (end 142.3359 116.9338) (width 0.3048) (layer "B.Cu") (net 4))
 (segment (start 142.3359 112.9191) (end 143.495 111.76) (width 0.3048) (layer "B.Cu") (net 4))
 (segment (start 142.3359 116.9338) (end 142.3359 112.9191) (width 0.3048) (layer "B.Cu") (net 4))
 (segment (start 146.05 120.65) (end 146.05 120.6479) (width 0.3048) (layer "B.Cu") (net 4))
 (segment (start 143.495 115.9741) (end 143.495 114.3) (width 0.3048) (layer "F.Cu") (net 5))
 (segment (start 138.43 119.38) (end 140.0891 119.38) (width 0.3048) (layer "F.Cu") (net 5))
 (segment (start 140.0891 119.38) (end 143.495 115.9741) (width 0.3048) (layer "F.Cu") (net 5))
 (segment (start 144.6 114.3) (end 143.495 114.3) (width 0.3048) (layer "B.Cu") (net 5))
 (segment (start 150.95 120.65) (end 144.6 114.3) (width 0.3048) (layer "B.Cu") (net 5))
 (segment (start 143.1209 85.09) (end 141.8618 86.3491) (width 0.3048) (layer "B.Cu") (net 8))
 (segment (start 133.7282 86.3491) (end 132.4691 85.09) (width 0.3048) (layer "B.Cu") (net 8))
 (segment (start 130.81 85.09) (end 132.4691 85.09) (width 0.3048) (layer "B.Cu") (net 8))
 (segment (start 141.8618 86.3491) (end 133.7282 86.3491) (width 0.3048) (layer "B.Cu") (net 8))
 (segment (start 144.78 85.09) (end 143.1209 85.09) (width 0.3048) (layer "B.Cu") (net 8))
 (segment (start 141.359 104.1401) (end 140.0891 105.41) (width 0.3048) (layer "B.Cu") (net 16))
 (segment (start 138.43 105.41) (end 140.0891 105.41) (width 0.3048) (layer "B.Cu") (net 16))
 (segment (start 152.4 105.41) (end 150.7409 105.41) (width 0.3048) (layer "B.Cu") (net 16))
 (segment (start 150.7409 105.41) (end 149.471 104.1401) (width 0.3048) (layer "B.Cu") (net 16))
 (segment (start 149.471 104.1401) (end 141.359 104.1401) (width 0.3048) (layer "B.Cu") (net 16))
 (segment (start 129.1528 125.3428) (end 130.81 127) (width 0.3048) (layer "F.Cu") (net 9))
 (segment (start 129.1528 89.2872) (end 129.1528 125.3428) (width 0.3048) (layer "F.Cu") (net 9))
 (segment (start 130.81 87.63) (end 129.1528 89.2872) (width 0.3048) (layer "F.Cu") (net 9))
 (segment (start 130.81 90.17) (end 132.4691 90.17) (width 0.3048) (layer "B.Cu") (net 10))
 (segment (start 140.2227 91.4399) (end 133.739 91.4399) (width 0.3048) (layer "B.Cu") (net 10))
 (segment (start 141.4926 90.17) (end 140.2227 91.4399) (width 0.3048) (layer "B.Cu") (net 10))
 (segment (start 144.78 90.17) (end 141.4926 90.17) (width 0.3048) (layer "B.Cu") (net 10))
 (segment (start 133.739 91.4399) (end 132.4691 90.17) (width 0.3048) (layer "B.Cu") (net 10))
 (segment (start 136.7709 106.6523) (end 137.1566 107.038) (width 0.3048) (layer "F.Cu") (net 18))
 (segment (start 136.7709 100.33) (end 136.7709 106.6523) (width 0.3048) (layer "F.Cu") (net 18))
 (segment (start 137.1566 113.63) (end 134.5709 116.2157) (width 0.3048) (layer "F.Cu") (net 18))
 (segment (start 134.5709 116.2157) (end 134.5709 123.1409) (width 0.3048) (layer "F.Cu") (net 18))
 (segment (start 137.1566 107.038) (end 137.1566 113.63) (width 0.3048) (layer "F.Cu") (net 18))
 (segment (start 138.43 100.33) (end 136.7709 100.33) (width 0.3048) (layer "F.Cu") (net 18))
 (via (at 134.5709 123.1409) (size 0.6858) (drill 0.3302) (layers "F.Cu" "B.Cu") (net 18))
 (segment (start 141.359 101.5999) (end 149.471 101.5999) (width 0.3048) (layer "B.Cu") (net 18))
 (segment (start 140.0891 100.33) (end 141.359 101.5999) (width 0.3048) (layer "B.Cu") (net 18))
 (segment (start 152.0036 100.33) (end 150.7409 100.33) (width 0.3048) (layer "B.Cu") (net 18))
 (segment (start 136.7709 125.3409) (end 134.5709 123.1409) (width 0.3048) (layer "B.Cu") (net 18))
 (segment (start 136.7709 127) (end 136.7709 125.3409) (width 0.3048) (layer "B.Cu") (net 18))
 (segment (start 138.43 100.33) (end 140.0891 100.33) (width 0.3048) (layer "B.Cu") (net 18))
 (segment (start 152.0036 100.33) (end 152.4 100.33) (width 0.3048) (layer "B.Cu") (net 18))
 (segment (start 138.43 127) (end 136.7709 127) (width 0.3048) (layer "B.Cu") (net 18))
 (segment (start 149.471 101.5999) (end 150.7409 100.33) (width 0.3048) (layer "B.Cu") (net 18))
 (segment (start 144.78 92.71) (end 143.1209 92.71) (width 0.3048) (layer "B.Cu") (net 11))
 (segment (start 139.9479 93.9799) (end 133.739 93.9799) (width 0.3048) (layer "B.Cu") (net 11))
 (segment (start 133.739 93.9799) (end 132.4691 92.71) (width 0.3048) (layer "B.Cu") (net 11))
 (segment (start 130.81 92.71) (end 132.4691 92.71) (width 0.3048) (layer "B.Cu") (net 11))
 (segment (start 141.2178 92.71) (end 139.9479 93.9799) (width 0.3048) (layer "B.Cu") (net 11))
 (segment (start 143.1209 92.71) (end 141.2178 92.71) (width 0.3048) (layer "B.Cu") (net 11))
 (segment (start 133.7391 96.52) (end 132.4691 95.25) (width 0.3048) (layer "B.Cu") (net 12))
 (segment (start 141.8509 96.52) (end 133.7391 96.52) (width 0.3048) (layer "B.Cu") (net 12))
 (segment (start 143.1209 95.25) (end 141.8509 96.52) (width 0.3048) (layer "B.Cu") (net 12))
 (segment (start 130.81 95.25) (end 132.4691 95.25) (width 0.3048) (layer "B.Cu") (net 12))
 (segment (start 144.78 95.25) (end 143.1209 95.25) (width 0.3048) (layer "B.Cu") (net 12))
 (segment (start 140.2897 94.7722) (end 140.1449 94.917) (width 0.3048) (layer "F.Cu") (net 13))
 (segment (start 140.1449 94.917) (end 140.1449 95.7186) (width 0.3048) (layer "F.Cu") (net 13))
 (segment (start 140.1449 95.7186) (end 139.3435 96.52) (width 0.3048) (layer "F.Cu") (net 13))
 (segment (start 139.3435 96.52) (end 133.7391 96.52) (width 0.3048) (layer "F.Cu") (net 13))
 (segment (start 133.7391 96.52) (end 132.4691 97.79) (width 0.3048) (layer "F.Cu") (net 13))
 (segment (start 130.81 97.79) (end 132.4691 97.79) (width 0.3048) (layer "F.Cu") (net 13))
 (via (at 140.2897 94.7722) (size 0.6858) (drill 0.3302) (layers "F.Cu" "B.Cu") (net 13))
 (segment (start 141.0822 93.9797) (end 140.2897 94.7722) (width 0.3048) (layer "B.Cu") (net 13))
 (segment (start 144.78 97.79) (end 146.4391 97.79) (width 0.3048) (layer "B.Cu") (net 13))
 (segment (start 146.4391 97.79) (end 146.4391 94.6946) (width 0.3048) (layer "B.Cu") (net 13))
 (segment (start 146.4391 94.6946) (end 145.7242 93.9797) (width 0.3048) (layer "B.Cu") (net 13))
 (segment (start 145.7242 93.9797) (end 141.0822 93.9797) (width 0.3048) (layer "B.Cu") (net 13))
 (segment (start 150.7409 92.71) (end 149.4709 91.44) (width 0.3048) (layer "B.Cu") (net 21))
 (segment (start 141.3591 91.44) (end 140.0891 92.71) (width 0.3048) (layer "B.Cu") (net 21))
 (segment (start 152.4 92.71) (end 150.7409 92.71) (width 0.3048) (layer "B.Cu") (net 21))
 (segment (start 149.4709 91.44) (end 141.3591 91.44) (width 0.3048) (layer "B.Cu") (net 21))
 (segment (start 138.43 92.71) (end 140.0891 92.71) (width 0.3048) (layer "B.Cu") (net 21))
 (segment (start 130.81 100.33) (end 132.4691 100.33) (width 0.3048) (layer "B.Cu") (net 14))
 (segment (start 141.851 99.0601) (end 133.739 99.0601) (width 0.3048) (layer "B.Cu") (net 14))
 (segment (start 144.78 100.33) (end 143.1209 100.33) (width 0.3048) (layer "B.Cu") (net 14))
 (segment (start 143.1209 100.33) (end 141.851 99.0601) (width 0.3048) (layer "B.Cu") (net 14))
 (segment (start 133.739 99.0601) (end 132.4691 100.33) (width 0.3048) (layer "B.Cu") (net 14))
 (segment (start 148.8774 79.3859) (end 133.8179 79.3859) (width 0.3048) (layer "B.Cu") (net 22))
 (segment (start 154.0591 84.5676) (end 148.8774 79.3859) (width 0.3048) (layer "B.Cu") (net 22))
 (segment (start 133.8179 79.3859) (end 129.1509 84.0529) (width 0.3048) (layer "B.Cu") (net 22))
 (segment (start 129.4301 86.36) (end 132.0924 86.36) (width 0.3048) (layer "B.Cu") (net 22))
 (segment (start 129.1509 86.0808) (end 129.4301 86.36) (width 0.3048) (layer "B.Cu") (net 22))
 (segment (start 132.0924 86.36) (end 135.9024 90.17) (width 0.3048) (layer "B.Cu") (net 22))
 (segment (start 152.4 90.17) (end 154.0591 90.17) (width 0.3048) (layer "B.Cu") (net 22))
 (segment (start 154.0591 90.17) (end 154.0591 84.5676) (width 0.3048) (layer "B.Cu") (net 22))
 (segment (start 135.9024 90.17) (end 138.43 90.17) (width 0.3048) (layer "B.Cu") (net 22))
 (segment (start 129.1509 84.0529) (end 129.1509 86.0808) (width 0.3048) (layer "B.Cu") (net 22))
 (segment (start 144.78 102.87) (end 141.4926 102.87) (width 0.3048) (layer "B.Cu") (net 15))
 (segment (start 141.4926 102.87) (end 140.2227 104.1399) (width 0.3048) (layer "B.Cu") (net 15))
 (segment (start 130.81 102.87) (end 132.4691 102.87) (width 0.3048) (layer "B.Cu") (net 15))
 (segment (start 133.739 104.1399) (end 132.4691 102.87) (width 0.3048) (layer "B.Cu") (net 15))
 (segment (start 140.2227 104.1399) (end 133.739 104.1399) (width 0.3048) (layer "B.Cu") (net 15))
 (segment (start 138.43 87.63) (end 140.0891 87.63) (width 0.3048) (layer "B.Cu") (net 23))
 (segment (start 149.471 88.8999) (end 141.359 88.8999) (width 0.3048) (layer "B.Cu") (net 23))
 (segment (start 141.359 88.8999) (end 140.0891 87.63) (width 0.3048) (layer "B.Cu") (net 23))
 (segment (start 152.4 87.63) (end 150.7409 87.63) (width 0.3048) (layer "B.Cu") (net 23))
 (segment (start 150.7409 87.63) (end 149.471 88.8999) (width 0.3048) (layer "B.Cu") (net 23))
 (segment (start 146.4391 105.9864) (end 146.4391 87.63) (width 0.3048) (layer "F.Cu") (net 24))
 (segment (start 132.4691 129.54) (end 135.3729 126.6362) (width 0.3048) (layer "F.Cu") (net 24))
 (segment (start 139.685 118.11) (end 141.446 116.349) (width 0.3048) (layer "F.Cu") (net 24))
 (segment (start 137.4597 118.11) (end 139.685 118.11) (width 0.3048) (layer "F.Cu") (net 24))
 (segment (start 135.3729 126.6362) (end 135.3729 120.1968) (width 0.3048) (layer "F.Cu") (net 24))
 (segment (start 135.3729 120.1968) (end 137.4597 118.11) (width 0.3048) (layer "F.Cu") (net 24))
 (segment (start 141.446 110.9795) (end 146.4391 105.9864) (width 0.3048) (layer "F.Cu") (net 24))
 (segment (start 141.446 116.349) (end 141.446 110.9795) (width 0.3048) (layer "F.Cu") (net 24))
 (segment (start 130.81 129.54) (end 132.4691 129.54) (width 0.3048) (layer "F.Cu") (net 24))
 (segment (start 144.78 87.63) (end 146.4391 87.63) (width 0.3048) (layer "F.Cu") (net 24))
 (segment (start 149.1747 119.2758) (end 149.1747 99.3562) (width 0.3048) (layer "F.Cu") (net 25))
 (segment (start 140.0891 129.54) (end 140.0891 128.3614) (width 0.3048) (layer "F.Cu") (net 25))
 (segment (start 140.0891 128.3614) (end 149.1747 119.2758) (width 0.3048) (layer "F.Cu") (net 25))
 (segment (start 138.43 129.54) (end 140.0891 129.54) (width 0.3048) (layer "F.Cu") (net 25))
 (segment (start 149.1747 99.3562) (end 150.7409 97.79) (width 0.3048) (layer "F.Cu") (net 25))
 (segment (start 152.4 97.79) (end 150.7409 97.79) (width 0.3048) (layer "F.Cu") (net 25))
 (segment (start 134.2309 132.08) (end 136.7709 129.54) (width 0.3048) (layer "B.Cu") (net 25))
 (segment (start 138.43 137.16) (end 136.7709 137.16) (width 0.3048) (layer "B.Cu") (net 25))
 (segment (start 137.6005 129.54) (end 136.7709 129.54) (width 0.3048) (layer "B.Cu") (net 25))
 (segment (start 137.6005 129.54) (end 138.0686 129.54) (width 0.3048) (layer "B.Cu") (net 25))
 (segment (start 130.81 132.08) (end 134.2309 132.08) (width 0.3048) (layer "B.Cu") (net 25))
 (segment (start 132.4691 124.46) (end 132.4691 125.2382) (width 0.3048) (layer "B.Cu") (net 25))
 (segment (start 138.43 129.54) (end 138.0686 129.54) (width 0.3048) (layer "B.Cu") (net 25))
 (segment (start 131.2065 124.46) (end 130.81 124.46) (width 0.3048) (layer "B.Cu") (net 25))
 (segment (start 134.2309 132.08) (end 134.2309 134.62) (width 0.3048) (layer "B.Cu") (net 25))
 (segment (start 134.2309 134.62) (end 136.7709 137.16) (width 0.3048) (layer "B.Cu") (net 25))
 (segment (start 132.4691 125.2382) (end 136.7709 129.54) (width 0.3048) (layer "B.Cu") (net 25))
 (segment (start 131.2065 124.46) (end 132.4691 124.46) (width 0.3048) (layer "B.Cu") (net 25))
 (segment (start 138.43 132.08) (end 140.0891 132.08) (width 0.3048) (layer "B.Cu") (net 26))
 (segment (start 154.0591 121.2374) (end 154.0591 95.25) (width 0.3048) (layer "B.Cu") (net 26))
 (segment (start 144.4756 130.8209) (end 154.0591 121.2374) (width 0.3048) (layer "B.Cu") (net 26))
 (segment (start 152.4 95.25) (end 154.0591 95.25) (width 0.3048) (layer "B.Cu") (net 26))
 (segment (start 141.3482 130.8209) (end 144.4756 130.8209) (width 0.3048) (layer "B.Cu") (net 26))
 (segment (start 140.0891 132.08) (end 141.3482 130.8209) (width 0.3048) (layer "B.Cu") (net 26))
 (segment (start 130.81 119.38) (end 132.4691 119.38) (width 0.3048) (layer "F.Cu") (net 27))
 (segment (start 132.4691 121.92) (end 132.4691 119.38) (width 0.3048) (layer "F.Cu") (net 27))
 (segment (start 130.81 121.92) (end 132.4691 121.92) (width 0.3048) (layer "F.Cu") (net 27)))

